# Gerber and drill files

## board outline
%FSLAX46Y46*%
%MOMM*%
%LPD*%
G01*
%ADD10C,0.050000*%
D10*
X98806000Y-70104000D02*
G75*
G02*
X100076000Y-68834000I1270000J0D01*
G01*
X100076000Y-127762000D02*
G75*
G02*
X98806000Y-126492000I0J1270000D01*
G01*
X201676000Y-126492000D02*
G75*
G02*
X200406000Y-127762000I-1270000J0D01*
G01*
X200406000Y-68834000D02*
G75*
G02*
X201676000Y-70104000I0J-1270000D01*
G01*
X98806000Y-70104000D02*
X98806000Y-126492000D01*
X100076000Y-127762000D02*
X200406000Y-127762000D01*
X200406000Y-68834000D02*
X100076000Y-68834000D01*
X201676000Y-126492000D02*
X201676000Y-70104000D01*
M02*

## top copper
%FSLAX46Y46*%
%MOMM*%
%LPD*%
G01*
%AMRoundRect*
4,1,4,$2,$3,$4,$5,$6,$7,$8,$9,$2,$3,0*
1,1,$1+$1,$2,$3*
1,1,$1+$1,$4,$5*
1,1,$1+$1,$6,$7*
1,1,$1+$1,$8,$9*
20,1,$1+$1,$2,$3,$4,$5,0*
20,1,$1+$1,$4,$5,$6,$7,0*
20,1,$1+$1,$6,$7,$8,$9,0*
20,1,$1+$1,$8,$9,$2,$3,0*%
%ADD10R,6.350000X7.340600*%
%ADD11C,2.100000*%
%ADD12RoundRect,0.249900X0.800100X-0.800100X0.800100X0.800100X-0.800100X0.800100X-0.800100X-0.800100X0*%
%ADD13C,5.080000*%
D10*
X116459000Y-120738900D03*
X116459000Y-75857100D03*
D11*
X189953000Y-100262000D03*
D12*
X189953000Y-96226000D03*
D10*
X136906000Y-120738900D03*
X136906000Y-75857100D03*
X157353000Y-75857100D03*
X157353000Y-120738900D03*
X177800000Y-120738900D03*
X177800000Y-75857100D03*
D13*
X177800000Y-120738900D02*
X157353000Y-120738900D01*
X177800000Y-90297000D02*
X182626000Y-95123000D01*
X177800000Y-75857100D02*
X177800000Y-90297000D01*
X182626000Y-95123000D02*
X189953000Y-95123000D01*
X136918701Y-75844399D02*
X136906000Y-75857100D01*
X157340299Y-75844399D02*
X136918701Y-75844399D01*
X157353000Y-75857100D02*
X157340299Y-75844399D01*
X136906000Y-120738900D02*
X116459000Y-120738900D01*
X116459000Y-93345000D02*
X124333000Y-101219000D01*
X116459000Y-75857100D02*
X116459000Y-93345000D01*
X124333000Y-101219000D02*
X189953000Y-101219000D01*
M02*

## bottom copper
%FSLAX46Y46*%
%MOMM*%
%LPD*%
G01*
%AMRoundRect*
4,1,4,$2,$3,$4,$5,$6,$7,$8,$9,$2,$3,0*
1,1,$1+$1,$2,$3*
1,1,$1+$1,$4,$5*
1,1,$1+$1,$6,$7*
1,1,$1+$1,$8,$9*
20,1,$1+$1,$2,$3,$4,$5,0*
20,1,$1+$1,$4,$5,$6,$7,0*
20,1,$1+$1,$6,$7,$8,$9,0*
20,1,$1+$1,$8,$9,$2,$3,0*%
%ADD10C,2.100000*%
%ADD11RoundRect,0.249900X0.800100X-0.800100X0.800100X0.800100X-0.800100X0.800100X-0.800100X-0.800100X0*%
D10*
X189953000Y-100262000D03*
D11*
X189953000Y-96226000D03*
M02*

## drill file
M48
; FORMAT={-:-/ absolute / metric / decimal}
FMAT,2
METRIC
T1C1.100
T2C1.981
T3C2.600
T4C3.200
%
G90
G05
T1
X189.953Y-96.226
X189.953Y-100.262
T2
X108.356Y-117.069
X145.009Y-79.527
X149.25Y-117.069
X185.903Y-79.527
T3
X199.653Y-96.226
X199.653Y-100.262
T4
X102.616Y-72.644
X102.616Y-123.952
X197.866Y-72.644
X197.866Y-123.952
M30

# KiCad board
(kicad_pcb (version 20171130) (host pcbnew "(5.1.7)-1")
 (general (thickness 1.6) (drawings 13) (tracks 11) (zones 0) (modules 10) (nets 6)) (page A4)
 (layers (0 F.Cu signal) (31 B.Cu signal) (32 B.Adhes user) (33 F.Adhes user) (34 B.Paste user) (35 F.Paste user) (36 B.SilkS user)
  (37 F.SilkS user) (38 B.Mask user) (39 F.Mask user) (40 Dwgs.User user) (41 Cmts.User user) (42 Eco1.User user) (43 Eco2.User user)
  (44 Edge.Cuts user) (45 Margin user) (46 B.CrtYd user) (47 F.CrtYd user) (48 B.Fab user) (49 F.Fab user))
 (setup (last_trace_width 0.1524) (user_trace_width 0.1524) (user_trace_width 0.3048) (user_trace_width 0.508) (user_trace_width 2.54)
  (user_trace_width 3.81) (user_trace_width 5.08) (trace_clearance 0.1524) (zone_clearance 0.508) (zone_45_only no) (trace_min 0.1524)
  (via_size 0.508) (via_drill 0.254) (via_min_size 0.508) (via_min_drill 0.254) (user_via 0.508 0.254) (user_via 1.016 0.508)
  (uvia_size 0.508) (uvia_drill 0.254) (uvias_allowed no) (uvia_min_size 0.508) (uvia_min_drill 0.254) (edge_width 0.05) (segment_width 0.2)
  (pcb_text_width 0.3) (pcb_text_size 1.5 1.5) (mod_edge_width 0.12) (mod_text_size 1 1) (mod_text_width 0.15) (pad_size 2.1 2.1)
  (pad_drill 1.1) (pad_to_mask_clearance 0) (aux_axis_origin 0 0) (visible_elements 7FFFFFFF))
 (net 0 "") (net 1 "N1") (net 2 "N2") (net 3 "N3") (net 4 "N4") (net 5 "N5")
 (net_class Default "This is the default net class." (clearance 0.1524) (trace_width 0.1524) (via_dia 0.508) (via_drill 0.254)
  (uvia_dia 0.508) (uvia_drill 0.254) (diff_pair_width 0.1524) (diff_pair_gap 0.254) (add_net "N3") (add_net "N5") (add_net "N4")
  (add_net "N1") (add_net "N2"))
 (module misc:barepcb (layer F.Cu) (at 147.066 130.048)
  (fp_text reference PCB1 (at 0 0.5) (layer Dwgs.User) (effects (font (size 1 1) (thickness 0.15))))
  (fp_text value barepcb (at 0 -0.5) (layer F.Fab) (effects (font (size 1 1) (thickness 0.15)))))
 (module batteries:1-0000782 (layer F.Cu) (at 116.459 98.298 90)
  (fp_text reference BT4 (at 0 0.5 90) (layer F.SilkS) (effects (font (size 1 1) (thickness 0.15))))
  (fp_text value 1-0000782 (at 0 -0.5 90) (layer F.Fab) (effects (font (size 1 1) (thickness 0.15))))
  (pad 1 smd rect (at -22.4409 0 90) (size 7.3406 6.35) (layers F.Cu F.Paste F.Mask) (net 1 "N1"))
  (pad 2 smd rect (at 22.4409 0 90) (size 7.3406 6.35) (layers F.Cu F.Paste F.Mask) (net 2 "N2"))
  (pad "" np_thru_hole circle (at -18.7706 -8.1026 90) (size 1.9812 1.9812) (drill 1.9812) (layers *.Cu *.Mask)))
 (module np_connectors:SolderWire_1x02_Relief (layer F.Cu) (at 189.357 98.298 90)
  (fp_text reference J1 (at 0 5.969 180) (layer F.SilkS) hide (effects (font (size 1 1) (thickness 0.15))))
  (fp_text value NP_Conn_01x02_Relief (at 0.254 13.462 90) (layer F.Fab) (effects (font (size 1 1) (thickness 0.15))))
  (pad "" np_thru_hole circle (at -1.964 10.296 90) (size 2.6 2.6) (drill 2.6) (layers *.Cu *.Mask))
  (pad 2 thru_hole circle (at -1.964 0.596 90) (size 2.1 2.1) (drill 1.1) (layers *.Cu *.Mask) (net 2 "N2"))
  (pad 1 thru_hole roundrect (at 2.072 0.596 90) (size 2.1 2.1) (drill 1.1) (layers *.Cu *.Mask) (roundrect_rratio 0.119) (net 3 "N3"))
  (pad "" np_thru_hole circle (at 2.072 10.296 90) (size 2.6 2.6) (drill 2.6) (layers *.Cu *.Mask)))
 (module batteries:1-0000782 (layer F.Cu) (at 136.906 98.298 270)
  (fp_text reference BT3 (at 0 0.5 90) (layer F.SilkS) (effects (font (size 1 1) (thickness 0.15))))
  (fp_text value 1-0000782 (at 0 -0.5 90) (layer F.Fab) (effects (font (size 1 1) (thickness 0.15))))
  (pad "" np_thru_hole circle (at -18.7706 -8.1026 270) (size 1.9812 1.9812) (drill 1.9812) (layers *.Cu *.Mask))
  (pad 2 smd rect (at 22.4409 0 270) (size 7.3406 6.35) (layers F.Cu F.Paste F.Mask) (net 1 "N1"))
  (pad 1 smd rect (at -22.4409 0 270) (size 7.3406 6.35) (layers F.Cu F.Paste F.Mask) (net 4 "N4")))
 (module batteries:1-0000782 (layer F.Cu) (at 157.353 98.298 90)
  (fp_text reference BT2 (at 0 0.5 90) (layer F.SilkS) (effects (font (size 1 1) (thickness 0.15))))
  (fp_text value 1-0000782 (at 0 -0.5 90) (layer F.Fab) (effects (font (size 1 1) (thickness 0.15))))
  (pad "" np_thru_hole circle (at -18.7706 -8.1026 90) (size 1.9812 1.9812) (drill 1.9812) (layers *.Cu *.Mask))
  (pad 2 smd rect (at 22.4409 0 90) (size 7.3406 6.35) (layers F.Cu F.Paste F.Mask) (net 4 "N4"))
  (pad 1 smd rect (at -22.4409 0 90) (size 7.3406 6.35) (layers F.Cu F.Paste F.Mask) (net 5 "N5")))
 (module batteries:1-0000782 (layer F.Cu) (at 177.8 98.298 270)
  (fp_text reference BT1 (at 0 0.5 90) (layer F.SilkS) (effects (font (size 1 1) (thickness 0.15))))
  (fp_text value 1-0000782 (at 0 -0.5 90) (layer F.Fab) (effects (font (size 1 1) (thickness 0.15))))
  (pad "" np_thru_hole circle (at -18.7706 -8.1026 270) (size 1.9812 1.9812) (drill 1.9812) (layers *.Cu *.Mask))
  (pad 2 smd rect (at 22.4409 0 270) (size 7.3406 6.35) (layers F.Cu F.Paste F.Mask) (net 5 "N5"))
  (pad 1 smd rect (at -22.4409 0 270) (size 7.3406 6.35) (layers F.Cu F.Paste F.Mask) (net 3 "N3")))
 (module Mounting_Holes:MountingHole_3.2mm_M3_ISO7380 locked (layer F.Cu) (at 102.616 72.644)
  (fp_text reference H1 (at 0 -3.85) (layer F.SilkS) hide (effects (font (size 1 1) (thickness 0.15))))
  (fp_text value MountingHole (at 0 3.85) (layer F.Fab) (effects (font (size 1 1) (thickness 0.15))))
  (pad 1 np_thru_hole circle (at 0 0) (size 3.2 3.2) (drill 3.2) (layers *.Cu *.Mask)))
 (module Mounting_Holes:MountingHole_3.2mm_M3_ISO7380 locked (layer F.Cu) (at 102.616 123.952)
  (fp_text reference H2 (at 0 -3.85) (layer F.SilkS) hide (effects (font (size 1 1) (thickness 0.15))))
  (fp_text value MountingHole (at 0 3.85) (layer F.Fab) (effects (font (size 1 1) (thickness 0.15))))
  (pad 1 np_thru_hole circle (at 0 0) (size 3.2 3.2) (drill 3.2) (layers *.Cu *.Mask)))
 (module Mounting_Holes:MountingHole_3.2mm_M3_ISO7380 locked (layer F.Cu) (at 197.866 72.644)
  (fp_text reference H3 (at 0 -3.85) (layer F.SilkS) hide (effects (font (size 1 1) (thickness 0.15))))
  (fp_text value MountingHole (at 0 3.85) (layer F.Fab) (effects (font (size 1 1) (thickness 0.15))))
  (pad 1 np_thru_hole circle (at 0 0) (size 3.2 3.2) (drill 3.2) (layers *.Cu *.Mask)))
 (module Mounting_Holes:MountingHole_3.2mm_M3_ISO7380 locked (layer F.Cu) (at 197.866 123.952)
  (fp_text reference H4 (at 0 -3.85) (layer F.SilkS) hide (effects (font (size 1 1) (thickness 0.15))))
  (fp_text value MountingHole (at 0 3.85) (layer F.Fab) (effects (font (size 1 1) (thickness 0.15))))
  (pad 1 np_thru_hole circle (at 0 0) (size 3.2 3.2) (drill 3.2) (layers *.Cu *.Mask)))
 (gr_arc (start 100.076 70.104) (end 100.076 68.834) (angle -90) (layer Edge.Cuts) (width 0.05))
 (gr_arc (start 100.076 126.492) (end 98.806 126.492) (angle -90) (layer Edge.Cuts) (width 0.05))
 (gr_arc (start 200.406 126.492) (end 200.406 127.762) (angle -90) (layer Edge.Cuts) (width 0.05))
 (gr_arc (start 200.406 70.104) (end 201.676 70.104) (angle -90) (layer Edge.Cuts) (width 0.05))
 (gr_line (start 98.806 70.104) (end 98.806 126.492) (layer Edge.Cuts) (width 0.05))
 (gr_line (start 100.076 127.762) (end 200.406 127.762) (layer Edge.Cuts) (width 0.05))
 (gr_line (start 200.406 68.834) (end 100.076 68.834) (layer Edge.Cuts) (width 0.05))
 (gr_line (start 201.676 126.492) (end 201.676 70.104) (layer Edge.Cuts) (width 0.05))
 (segment (start 177.8 120.7389) (end 157.353 120.7389) (width 5.08) (layer F.Cu) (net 5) (status 30))
 (segment (start 177.8 90.297) (end 182.626 95.123) (width 5.08) (layer F.Cu) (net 3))
 (segment (start 177.8 75.8571) (end 177.8 90.297) (width 5.08) (layer F.Cu) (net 3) (status 10))
 (segment (start 182.626 95.123) (end 189.953 95.123) (width 5.08) (layer F.Cu) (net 3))
 (segment (start 136.918701 75.844399) (end 136.906 75.8571) (width 5.08) (layer F.Cu) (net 4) (status 30))
 (segment (start 157.340299 75.844399) (end 136.918701 75.844399) (width 5.08) (layer F.Cu) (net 4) (status 30))
 (segment (start 157.353 75.8571) (end 157.340299 75.844399) (width 5.08) (layer F.Cu) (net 4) (status 30))
 (segment (start 136.906 120.7389) (end 116.459 120.7389) (width 5.08) (layer F.Cu) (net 1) (status 30))
 (segment (start 116.459 93.345) (end 124.333 101.219) (width 5.08) (layer F.Cu) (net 2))
 (segment (start 116.459 75.8571) (end 116.459 93.345) (width 5.08) (layer F.Cu) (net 2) (status 10))
 (segment (start 124.333 101.219) (end 189.953 101.219) (width 5.08) (layer F.Cu) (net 2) (status 20)))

